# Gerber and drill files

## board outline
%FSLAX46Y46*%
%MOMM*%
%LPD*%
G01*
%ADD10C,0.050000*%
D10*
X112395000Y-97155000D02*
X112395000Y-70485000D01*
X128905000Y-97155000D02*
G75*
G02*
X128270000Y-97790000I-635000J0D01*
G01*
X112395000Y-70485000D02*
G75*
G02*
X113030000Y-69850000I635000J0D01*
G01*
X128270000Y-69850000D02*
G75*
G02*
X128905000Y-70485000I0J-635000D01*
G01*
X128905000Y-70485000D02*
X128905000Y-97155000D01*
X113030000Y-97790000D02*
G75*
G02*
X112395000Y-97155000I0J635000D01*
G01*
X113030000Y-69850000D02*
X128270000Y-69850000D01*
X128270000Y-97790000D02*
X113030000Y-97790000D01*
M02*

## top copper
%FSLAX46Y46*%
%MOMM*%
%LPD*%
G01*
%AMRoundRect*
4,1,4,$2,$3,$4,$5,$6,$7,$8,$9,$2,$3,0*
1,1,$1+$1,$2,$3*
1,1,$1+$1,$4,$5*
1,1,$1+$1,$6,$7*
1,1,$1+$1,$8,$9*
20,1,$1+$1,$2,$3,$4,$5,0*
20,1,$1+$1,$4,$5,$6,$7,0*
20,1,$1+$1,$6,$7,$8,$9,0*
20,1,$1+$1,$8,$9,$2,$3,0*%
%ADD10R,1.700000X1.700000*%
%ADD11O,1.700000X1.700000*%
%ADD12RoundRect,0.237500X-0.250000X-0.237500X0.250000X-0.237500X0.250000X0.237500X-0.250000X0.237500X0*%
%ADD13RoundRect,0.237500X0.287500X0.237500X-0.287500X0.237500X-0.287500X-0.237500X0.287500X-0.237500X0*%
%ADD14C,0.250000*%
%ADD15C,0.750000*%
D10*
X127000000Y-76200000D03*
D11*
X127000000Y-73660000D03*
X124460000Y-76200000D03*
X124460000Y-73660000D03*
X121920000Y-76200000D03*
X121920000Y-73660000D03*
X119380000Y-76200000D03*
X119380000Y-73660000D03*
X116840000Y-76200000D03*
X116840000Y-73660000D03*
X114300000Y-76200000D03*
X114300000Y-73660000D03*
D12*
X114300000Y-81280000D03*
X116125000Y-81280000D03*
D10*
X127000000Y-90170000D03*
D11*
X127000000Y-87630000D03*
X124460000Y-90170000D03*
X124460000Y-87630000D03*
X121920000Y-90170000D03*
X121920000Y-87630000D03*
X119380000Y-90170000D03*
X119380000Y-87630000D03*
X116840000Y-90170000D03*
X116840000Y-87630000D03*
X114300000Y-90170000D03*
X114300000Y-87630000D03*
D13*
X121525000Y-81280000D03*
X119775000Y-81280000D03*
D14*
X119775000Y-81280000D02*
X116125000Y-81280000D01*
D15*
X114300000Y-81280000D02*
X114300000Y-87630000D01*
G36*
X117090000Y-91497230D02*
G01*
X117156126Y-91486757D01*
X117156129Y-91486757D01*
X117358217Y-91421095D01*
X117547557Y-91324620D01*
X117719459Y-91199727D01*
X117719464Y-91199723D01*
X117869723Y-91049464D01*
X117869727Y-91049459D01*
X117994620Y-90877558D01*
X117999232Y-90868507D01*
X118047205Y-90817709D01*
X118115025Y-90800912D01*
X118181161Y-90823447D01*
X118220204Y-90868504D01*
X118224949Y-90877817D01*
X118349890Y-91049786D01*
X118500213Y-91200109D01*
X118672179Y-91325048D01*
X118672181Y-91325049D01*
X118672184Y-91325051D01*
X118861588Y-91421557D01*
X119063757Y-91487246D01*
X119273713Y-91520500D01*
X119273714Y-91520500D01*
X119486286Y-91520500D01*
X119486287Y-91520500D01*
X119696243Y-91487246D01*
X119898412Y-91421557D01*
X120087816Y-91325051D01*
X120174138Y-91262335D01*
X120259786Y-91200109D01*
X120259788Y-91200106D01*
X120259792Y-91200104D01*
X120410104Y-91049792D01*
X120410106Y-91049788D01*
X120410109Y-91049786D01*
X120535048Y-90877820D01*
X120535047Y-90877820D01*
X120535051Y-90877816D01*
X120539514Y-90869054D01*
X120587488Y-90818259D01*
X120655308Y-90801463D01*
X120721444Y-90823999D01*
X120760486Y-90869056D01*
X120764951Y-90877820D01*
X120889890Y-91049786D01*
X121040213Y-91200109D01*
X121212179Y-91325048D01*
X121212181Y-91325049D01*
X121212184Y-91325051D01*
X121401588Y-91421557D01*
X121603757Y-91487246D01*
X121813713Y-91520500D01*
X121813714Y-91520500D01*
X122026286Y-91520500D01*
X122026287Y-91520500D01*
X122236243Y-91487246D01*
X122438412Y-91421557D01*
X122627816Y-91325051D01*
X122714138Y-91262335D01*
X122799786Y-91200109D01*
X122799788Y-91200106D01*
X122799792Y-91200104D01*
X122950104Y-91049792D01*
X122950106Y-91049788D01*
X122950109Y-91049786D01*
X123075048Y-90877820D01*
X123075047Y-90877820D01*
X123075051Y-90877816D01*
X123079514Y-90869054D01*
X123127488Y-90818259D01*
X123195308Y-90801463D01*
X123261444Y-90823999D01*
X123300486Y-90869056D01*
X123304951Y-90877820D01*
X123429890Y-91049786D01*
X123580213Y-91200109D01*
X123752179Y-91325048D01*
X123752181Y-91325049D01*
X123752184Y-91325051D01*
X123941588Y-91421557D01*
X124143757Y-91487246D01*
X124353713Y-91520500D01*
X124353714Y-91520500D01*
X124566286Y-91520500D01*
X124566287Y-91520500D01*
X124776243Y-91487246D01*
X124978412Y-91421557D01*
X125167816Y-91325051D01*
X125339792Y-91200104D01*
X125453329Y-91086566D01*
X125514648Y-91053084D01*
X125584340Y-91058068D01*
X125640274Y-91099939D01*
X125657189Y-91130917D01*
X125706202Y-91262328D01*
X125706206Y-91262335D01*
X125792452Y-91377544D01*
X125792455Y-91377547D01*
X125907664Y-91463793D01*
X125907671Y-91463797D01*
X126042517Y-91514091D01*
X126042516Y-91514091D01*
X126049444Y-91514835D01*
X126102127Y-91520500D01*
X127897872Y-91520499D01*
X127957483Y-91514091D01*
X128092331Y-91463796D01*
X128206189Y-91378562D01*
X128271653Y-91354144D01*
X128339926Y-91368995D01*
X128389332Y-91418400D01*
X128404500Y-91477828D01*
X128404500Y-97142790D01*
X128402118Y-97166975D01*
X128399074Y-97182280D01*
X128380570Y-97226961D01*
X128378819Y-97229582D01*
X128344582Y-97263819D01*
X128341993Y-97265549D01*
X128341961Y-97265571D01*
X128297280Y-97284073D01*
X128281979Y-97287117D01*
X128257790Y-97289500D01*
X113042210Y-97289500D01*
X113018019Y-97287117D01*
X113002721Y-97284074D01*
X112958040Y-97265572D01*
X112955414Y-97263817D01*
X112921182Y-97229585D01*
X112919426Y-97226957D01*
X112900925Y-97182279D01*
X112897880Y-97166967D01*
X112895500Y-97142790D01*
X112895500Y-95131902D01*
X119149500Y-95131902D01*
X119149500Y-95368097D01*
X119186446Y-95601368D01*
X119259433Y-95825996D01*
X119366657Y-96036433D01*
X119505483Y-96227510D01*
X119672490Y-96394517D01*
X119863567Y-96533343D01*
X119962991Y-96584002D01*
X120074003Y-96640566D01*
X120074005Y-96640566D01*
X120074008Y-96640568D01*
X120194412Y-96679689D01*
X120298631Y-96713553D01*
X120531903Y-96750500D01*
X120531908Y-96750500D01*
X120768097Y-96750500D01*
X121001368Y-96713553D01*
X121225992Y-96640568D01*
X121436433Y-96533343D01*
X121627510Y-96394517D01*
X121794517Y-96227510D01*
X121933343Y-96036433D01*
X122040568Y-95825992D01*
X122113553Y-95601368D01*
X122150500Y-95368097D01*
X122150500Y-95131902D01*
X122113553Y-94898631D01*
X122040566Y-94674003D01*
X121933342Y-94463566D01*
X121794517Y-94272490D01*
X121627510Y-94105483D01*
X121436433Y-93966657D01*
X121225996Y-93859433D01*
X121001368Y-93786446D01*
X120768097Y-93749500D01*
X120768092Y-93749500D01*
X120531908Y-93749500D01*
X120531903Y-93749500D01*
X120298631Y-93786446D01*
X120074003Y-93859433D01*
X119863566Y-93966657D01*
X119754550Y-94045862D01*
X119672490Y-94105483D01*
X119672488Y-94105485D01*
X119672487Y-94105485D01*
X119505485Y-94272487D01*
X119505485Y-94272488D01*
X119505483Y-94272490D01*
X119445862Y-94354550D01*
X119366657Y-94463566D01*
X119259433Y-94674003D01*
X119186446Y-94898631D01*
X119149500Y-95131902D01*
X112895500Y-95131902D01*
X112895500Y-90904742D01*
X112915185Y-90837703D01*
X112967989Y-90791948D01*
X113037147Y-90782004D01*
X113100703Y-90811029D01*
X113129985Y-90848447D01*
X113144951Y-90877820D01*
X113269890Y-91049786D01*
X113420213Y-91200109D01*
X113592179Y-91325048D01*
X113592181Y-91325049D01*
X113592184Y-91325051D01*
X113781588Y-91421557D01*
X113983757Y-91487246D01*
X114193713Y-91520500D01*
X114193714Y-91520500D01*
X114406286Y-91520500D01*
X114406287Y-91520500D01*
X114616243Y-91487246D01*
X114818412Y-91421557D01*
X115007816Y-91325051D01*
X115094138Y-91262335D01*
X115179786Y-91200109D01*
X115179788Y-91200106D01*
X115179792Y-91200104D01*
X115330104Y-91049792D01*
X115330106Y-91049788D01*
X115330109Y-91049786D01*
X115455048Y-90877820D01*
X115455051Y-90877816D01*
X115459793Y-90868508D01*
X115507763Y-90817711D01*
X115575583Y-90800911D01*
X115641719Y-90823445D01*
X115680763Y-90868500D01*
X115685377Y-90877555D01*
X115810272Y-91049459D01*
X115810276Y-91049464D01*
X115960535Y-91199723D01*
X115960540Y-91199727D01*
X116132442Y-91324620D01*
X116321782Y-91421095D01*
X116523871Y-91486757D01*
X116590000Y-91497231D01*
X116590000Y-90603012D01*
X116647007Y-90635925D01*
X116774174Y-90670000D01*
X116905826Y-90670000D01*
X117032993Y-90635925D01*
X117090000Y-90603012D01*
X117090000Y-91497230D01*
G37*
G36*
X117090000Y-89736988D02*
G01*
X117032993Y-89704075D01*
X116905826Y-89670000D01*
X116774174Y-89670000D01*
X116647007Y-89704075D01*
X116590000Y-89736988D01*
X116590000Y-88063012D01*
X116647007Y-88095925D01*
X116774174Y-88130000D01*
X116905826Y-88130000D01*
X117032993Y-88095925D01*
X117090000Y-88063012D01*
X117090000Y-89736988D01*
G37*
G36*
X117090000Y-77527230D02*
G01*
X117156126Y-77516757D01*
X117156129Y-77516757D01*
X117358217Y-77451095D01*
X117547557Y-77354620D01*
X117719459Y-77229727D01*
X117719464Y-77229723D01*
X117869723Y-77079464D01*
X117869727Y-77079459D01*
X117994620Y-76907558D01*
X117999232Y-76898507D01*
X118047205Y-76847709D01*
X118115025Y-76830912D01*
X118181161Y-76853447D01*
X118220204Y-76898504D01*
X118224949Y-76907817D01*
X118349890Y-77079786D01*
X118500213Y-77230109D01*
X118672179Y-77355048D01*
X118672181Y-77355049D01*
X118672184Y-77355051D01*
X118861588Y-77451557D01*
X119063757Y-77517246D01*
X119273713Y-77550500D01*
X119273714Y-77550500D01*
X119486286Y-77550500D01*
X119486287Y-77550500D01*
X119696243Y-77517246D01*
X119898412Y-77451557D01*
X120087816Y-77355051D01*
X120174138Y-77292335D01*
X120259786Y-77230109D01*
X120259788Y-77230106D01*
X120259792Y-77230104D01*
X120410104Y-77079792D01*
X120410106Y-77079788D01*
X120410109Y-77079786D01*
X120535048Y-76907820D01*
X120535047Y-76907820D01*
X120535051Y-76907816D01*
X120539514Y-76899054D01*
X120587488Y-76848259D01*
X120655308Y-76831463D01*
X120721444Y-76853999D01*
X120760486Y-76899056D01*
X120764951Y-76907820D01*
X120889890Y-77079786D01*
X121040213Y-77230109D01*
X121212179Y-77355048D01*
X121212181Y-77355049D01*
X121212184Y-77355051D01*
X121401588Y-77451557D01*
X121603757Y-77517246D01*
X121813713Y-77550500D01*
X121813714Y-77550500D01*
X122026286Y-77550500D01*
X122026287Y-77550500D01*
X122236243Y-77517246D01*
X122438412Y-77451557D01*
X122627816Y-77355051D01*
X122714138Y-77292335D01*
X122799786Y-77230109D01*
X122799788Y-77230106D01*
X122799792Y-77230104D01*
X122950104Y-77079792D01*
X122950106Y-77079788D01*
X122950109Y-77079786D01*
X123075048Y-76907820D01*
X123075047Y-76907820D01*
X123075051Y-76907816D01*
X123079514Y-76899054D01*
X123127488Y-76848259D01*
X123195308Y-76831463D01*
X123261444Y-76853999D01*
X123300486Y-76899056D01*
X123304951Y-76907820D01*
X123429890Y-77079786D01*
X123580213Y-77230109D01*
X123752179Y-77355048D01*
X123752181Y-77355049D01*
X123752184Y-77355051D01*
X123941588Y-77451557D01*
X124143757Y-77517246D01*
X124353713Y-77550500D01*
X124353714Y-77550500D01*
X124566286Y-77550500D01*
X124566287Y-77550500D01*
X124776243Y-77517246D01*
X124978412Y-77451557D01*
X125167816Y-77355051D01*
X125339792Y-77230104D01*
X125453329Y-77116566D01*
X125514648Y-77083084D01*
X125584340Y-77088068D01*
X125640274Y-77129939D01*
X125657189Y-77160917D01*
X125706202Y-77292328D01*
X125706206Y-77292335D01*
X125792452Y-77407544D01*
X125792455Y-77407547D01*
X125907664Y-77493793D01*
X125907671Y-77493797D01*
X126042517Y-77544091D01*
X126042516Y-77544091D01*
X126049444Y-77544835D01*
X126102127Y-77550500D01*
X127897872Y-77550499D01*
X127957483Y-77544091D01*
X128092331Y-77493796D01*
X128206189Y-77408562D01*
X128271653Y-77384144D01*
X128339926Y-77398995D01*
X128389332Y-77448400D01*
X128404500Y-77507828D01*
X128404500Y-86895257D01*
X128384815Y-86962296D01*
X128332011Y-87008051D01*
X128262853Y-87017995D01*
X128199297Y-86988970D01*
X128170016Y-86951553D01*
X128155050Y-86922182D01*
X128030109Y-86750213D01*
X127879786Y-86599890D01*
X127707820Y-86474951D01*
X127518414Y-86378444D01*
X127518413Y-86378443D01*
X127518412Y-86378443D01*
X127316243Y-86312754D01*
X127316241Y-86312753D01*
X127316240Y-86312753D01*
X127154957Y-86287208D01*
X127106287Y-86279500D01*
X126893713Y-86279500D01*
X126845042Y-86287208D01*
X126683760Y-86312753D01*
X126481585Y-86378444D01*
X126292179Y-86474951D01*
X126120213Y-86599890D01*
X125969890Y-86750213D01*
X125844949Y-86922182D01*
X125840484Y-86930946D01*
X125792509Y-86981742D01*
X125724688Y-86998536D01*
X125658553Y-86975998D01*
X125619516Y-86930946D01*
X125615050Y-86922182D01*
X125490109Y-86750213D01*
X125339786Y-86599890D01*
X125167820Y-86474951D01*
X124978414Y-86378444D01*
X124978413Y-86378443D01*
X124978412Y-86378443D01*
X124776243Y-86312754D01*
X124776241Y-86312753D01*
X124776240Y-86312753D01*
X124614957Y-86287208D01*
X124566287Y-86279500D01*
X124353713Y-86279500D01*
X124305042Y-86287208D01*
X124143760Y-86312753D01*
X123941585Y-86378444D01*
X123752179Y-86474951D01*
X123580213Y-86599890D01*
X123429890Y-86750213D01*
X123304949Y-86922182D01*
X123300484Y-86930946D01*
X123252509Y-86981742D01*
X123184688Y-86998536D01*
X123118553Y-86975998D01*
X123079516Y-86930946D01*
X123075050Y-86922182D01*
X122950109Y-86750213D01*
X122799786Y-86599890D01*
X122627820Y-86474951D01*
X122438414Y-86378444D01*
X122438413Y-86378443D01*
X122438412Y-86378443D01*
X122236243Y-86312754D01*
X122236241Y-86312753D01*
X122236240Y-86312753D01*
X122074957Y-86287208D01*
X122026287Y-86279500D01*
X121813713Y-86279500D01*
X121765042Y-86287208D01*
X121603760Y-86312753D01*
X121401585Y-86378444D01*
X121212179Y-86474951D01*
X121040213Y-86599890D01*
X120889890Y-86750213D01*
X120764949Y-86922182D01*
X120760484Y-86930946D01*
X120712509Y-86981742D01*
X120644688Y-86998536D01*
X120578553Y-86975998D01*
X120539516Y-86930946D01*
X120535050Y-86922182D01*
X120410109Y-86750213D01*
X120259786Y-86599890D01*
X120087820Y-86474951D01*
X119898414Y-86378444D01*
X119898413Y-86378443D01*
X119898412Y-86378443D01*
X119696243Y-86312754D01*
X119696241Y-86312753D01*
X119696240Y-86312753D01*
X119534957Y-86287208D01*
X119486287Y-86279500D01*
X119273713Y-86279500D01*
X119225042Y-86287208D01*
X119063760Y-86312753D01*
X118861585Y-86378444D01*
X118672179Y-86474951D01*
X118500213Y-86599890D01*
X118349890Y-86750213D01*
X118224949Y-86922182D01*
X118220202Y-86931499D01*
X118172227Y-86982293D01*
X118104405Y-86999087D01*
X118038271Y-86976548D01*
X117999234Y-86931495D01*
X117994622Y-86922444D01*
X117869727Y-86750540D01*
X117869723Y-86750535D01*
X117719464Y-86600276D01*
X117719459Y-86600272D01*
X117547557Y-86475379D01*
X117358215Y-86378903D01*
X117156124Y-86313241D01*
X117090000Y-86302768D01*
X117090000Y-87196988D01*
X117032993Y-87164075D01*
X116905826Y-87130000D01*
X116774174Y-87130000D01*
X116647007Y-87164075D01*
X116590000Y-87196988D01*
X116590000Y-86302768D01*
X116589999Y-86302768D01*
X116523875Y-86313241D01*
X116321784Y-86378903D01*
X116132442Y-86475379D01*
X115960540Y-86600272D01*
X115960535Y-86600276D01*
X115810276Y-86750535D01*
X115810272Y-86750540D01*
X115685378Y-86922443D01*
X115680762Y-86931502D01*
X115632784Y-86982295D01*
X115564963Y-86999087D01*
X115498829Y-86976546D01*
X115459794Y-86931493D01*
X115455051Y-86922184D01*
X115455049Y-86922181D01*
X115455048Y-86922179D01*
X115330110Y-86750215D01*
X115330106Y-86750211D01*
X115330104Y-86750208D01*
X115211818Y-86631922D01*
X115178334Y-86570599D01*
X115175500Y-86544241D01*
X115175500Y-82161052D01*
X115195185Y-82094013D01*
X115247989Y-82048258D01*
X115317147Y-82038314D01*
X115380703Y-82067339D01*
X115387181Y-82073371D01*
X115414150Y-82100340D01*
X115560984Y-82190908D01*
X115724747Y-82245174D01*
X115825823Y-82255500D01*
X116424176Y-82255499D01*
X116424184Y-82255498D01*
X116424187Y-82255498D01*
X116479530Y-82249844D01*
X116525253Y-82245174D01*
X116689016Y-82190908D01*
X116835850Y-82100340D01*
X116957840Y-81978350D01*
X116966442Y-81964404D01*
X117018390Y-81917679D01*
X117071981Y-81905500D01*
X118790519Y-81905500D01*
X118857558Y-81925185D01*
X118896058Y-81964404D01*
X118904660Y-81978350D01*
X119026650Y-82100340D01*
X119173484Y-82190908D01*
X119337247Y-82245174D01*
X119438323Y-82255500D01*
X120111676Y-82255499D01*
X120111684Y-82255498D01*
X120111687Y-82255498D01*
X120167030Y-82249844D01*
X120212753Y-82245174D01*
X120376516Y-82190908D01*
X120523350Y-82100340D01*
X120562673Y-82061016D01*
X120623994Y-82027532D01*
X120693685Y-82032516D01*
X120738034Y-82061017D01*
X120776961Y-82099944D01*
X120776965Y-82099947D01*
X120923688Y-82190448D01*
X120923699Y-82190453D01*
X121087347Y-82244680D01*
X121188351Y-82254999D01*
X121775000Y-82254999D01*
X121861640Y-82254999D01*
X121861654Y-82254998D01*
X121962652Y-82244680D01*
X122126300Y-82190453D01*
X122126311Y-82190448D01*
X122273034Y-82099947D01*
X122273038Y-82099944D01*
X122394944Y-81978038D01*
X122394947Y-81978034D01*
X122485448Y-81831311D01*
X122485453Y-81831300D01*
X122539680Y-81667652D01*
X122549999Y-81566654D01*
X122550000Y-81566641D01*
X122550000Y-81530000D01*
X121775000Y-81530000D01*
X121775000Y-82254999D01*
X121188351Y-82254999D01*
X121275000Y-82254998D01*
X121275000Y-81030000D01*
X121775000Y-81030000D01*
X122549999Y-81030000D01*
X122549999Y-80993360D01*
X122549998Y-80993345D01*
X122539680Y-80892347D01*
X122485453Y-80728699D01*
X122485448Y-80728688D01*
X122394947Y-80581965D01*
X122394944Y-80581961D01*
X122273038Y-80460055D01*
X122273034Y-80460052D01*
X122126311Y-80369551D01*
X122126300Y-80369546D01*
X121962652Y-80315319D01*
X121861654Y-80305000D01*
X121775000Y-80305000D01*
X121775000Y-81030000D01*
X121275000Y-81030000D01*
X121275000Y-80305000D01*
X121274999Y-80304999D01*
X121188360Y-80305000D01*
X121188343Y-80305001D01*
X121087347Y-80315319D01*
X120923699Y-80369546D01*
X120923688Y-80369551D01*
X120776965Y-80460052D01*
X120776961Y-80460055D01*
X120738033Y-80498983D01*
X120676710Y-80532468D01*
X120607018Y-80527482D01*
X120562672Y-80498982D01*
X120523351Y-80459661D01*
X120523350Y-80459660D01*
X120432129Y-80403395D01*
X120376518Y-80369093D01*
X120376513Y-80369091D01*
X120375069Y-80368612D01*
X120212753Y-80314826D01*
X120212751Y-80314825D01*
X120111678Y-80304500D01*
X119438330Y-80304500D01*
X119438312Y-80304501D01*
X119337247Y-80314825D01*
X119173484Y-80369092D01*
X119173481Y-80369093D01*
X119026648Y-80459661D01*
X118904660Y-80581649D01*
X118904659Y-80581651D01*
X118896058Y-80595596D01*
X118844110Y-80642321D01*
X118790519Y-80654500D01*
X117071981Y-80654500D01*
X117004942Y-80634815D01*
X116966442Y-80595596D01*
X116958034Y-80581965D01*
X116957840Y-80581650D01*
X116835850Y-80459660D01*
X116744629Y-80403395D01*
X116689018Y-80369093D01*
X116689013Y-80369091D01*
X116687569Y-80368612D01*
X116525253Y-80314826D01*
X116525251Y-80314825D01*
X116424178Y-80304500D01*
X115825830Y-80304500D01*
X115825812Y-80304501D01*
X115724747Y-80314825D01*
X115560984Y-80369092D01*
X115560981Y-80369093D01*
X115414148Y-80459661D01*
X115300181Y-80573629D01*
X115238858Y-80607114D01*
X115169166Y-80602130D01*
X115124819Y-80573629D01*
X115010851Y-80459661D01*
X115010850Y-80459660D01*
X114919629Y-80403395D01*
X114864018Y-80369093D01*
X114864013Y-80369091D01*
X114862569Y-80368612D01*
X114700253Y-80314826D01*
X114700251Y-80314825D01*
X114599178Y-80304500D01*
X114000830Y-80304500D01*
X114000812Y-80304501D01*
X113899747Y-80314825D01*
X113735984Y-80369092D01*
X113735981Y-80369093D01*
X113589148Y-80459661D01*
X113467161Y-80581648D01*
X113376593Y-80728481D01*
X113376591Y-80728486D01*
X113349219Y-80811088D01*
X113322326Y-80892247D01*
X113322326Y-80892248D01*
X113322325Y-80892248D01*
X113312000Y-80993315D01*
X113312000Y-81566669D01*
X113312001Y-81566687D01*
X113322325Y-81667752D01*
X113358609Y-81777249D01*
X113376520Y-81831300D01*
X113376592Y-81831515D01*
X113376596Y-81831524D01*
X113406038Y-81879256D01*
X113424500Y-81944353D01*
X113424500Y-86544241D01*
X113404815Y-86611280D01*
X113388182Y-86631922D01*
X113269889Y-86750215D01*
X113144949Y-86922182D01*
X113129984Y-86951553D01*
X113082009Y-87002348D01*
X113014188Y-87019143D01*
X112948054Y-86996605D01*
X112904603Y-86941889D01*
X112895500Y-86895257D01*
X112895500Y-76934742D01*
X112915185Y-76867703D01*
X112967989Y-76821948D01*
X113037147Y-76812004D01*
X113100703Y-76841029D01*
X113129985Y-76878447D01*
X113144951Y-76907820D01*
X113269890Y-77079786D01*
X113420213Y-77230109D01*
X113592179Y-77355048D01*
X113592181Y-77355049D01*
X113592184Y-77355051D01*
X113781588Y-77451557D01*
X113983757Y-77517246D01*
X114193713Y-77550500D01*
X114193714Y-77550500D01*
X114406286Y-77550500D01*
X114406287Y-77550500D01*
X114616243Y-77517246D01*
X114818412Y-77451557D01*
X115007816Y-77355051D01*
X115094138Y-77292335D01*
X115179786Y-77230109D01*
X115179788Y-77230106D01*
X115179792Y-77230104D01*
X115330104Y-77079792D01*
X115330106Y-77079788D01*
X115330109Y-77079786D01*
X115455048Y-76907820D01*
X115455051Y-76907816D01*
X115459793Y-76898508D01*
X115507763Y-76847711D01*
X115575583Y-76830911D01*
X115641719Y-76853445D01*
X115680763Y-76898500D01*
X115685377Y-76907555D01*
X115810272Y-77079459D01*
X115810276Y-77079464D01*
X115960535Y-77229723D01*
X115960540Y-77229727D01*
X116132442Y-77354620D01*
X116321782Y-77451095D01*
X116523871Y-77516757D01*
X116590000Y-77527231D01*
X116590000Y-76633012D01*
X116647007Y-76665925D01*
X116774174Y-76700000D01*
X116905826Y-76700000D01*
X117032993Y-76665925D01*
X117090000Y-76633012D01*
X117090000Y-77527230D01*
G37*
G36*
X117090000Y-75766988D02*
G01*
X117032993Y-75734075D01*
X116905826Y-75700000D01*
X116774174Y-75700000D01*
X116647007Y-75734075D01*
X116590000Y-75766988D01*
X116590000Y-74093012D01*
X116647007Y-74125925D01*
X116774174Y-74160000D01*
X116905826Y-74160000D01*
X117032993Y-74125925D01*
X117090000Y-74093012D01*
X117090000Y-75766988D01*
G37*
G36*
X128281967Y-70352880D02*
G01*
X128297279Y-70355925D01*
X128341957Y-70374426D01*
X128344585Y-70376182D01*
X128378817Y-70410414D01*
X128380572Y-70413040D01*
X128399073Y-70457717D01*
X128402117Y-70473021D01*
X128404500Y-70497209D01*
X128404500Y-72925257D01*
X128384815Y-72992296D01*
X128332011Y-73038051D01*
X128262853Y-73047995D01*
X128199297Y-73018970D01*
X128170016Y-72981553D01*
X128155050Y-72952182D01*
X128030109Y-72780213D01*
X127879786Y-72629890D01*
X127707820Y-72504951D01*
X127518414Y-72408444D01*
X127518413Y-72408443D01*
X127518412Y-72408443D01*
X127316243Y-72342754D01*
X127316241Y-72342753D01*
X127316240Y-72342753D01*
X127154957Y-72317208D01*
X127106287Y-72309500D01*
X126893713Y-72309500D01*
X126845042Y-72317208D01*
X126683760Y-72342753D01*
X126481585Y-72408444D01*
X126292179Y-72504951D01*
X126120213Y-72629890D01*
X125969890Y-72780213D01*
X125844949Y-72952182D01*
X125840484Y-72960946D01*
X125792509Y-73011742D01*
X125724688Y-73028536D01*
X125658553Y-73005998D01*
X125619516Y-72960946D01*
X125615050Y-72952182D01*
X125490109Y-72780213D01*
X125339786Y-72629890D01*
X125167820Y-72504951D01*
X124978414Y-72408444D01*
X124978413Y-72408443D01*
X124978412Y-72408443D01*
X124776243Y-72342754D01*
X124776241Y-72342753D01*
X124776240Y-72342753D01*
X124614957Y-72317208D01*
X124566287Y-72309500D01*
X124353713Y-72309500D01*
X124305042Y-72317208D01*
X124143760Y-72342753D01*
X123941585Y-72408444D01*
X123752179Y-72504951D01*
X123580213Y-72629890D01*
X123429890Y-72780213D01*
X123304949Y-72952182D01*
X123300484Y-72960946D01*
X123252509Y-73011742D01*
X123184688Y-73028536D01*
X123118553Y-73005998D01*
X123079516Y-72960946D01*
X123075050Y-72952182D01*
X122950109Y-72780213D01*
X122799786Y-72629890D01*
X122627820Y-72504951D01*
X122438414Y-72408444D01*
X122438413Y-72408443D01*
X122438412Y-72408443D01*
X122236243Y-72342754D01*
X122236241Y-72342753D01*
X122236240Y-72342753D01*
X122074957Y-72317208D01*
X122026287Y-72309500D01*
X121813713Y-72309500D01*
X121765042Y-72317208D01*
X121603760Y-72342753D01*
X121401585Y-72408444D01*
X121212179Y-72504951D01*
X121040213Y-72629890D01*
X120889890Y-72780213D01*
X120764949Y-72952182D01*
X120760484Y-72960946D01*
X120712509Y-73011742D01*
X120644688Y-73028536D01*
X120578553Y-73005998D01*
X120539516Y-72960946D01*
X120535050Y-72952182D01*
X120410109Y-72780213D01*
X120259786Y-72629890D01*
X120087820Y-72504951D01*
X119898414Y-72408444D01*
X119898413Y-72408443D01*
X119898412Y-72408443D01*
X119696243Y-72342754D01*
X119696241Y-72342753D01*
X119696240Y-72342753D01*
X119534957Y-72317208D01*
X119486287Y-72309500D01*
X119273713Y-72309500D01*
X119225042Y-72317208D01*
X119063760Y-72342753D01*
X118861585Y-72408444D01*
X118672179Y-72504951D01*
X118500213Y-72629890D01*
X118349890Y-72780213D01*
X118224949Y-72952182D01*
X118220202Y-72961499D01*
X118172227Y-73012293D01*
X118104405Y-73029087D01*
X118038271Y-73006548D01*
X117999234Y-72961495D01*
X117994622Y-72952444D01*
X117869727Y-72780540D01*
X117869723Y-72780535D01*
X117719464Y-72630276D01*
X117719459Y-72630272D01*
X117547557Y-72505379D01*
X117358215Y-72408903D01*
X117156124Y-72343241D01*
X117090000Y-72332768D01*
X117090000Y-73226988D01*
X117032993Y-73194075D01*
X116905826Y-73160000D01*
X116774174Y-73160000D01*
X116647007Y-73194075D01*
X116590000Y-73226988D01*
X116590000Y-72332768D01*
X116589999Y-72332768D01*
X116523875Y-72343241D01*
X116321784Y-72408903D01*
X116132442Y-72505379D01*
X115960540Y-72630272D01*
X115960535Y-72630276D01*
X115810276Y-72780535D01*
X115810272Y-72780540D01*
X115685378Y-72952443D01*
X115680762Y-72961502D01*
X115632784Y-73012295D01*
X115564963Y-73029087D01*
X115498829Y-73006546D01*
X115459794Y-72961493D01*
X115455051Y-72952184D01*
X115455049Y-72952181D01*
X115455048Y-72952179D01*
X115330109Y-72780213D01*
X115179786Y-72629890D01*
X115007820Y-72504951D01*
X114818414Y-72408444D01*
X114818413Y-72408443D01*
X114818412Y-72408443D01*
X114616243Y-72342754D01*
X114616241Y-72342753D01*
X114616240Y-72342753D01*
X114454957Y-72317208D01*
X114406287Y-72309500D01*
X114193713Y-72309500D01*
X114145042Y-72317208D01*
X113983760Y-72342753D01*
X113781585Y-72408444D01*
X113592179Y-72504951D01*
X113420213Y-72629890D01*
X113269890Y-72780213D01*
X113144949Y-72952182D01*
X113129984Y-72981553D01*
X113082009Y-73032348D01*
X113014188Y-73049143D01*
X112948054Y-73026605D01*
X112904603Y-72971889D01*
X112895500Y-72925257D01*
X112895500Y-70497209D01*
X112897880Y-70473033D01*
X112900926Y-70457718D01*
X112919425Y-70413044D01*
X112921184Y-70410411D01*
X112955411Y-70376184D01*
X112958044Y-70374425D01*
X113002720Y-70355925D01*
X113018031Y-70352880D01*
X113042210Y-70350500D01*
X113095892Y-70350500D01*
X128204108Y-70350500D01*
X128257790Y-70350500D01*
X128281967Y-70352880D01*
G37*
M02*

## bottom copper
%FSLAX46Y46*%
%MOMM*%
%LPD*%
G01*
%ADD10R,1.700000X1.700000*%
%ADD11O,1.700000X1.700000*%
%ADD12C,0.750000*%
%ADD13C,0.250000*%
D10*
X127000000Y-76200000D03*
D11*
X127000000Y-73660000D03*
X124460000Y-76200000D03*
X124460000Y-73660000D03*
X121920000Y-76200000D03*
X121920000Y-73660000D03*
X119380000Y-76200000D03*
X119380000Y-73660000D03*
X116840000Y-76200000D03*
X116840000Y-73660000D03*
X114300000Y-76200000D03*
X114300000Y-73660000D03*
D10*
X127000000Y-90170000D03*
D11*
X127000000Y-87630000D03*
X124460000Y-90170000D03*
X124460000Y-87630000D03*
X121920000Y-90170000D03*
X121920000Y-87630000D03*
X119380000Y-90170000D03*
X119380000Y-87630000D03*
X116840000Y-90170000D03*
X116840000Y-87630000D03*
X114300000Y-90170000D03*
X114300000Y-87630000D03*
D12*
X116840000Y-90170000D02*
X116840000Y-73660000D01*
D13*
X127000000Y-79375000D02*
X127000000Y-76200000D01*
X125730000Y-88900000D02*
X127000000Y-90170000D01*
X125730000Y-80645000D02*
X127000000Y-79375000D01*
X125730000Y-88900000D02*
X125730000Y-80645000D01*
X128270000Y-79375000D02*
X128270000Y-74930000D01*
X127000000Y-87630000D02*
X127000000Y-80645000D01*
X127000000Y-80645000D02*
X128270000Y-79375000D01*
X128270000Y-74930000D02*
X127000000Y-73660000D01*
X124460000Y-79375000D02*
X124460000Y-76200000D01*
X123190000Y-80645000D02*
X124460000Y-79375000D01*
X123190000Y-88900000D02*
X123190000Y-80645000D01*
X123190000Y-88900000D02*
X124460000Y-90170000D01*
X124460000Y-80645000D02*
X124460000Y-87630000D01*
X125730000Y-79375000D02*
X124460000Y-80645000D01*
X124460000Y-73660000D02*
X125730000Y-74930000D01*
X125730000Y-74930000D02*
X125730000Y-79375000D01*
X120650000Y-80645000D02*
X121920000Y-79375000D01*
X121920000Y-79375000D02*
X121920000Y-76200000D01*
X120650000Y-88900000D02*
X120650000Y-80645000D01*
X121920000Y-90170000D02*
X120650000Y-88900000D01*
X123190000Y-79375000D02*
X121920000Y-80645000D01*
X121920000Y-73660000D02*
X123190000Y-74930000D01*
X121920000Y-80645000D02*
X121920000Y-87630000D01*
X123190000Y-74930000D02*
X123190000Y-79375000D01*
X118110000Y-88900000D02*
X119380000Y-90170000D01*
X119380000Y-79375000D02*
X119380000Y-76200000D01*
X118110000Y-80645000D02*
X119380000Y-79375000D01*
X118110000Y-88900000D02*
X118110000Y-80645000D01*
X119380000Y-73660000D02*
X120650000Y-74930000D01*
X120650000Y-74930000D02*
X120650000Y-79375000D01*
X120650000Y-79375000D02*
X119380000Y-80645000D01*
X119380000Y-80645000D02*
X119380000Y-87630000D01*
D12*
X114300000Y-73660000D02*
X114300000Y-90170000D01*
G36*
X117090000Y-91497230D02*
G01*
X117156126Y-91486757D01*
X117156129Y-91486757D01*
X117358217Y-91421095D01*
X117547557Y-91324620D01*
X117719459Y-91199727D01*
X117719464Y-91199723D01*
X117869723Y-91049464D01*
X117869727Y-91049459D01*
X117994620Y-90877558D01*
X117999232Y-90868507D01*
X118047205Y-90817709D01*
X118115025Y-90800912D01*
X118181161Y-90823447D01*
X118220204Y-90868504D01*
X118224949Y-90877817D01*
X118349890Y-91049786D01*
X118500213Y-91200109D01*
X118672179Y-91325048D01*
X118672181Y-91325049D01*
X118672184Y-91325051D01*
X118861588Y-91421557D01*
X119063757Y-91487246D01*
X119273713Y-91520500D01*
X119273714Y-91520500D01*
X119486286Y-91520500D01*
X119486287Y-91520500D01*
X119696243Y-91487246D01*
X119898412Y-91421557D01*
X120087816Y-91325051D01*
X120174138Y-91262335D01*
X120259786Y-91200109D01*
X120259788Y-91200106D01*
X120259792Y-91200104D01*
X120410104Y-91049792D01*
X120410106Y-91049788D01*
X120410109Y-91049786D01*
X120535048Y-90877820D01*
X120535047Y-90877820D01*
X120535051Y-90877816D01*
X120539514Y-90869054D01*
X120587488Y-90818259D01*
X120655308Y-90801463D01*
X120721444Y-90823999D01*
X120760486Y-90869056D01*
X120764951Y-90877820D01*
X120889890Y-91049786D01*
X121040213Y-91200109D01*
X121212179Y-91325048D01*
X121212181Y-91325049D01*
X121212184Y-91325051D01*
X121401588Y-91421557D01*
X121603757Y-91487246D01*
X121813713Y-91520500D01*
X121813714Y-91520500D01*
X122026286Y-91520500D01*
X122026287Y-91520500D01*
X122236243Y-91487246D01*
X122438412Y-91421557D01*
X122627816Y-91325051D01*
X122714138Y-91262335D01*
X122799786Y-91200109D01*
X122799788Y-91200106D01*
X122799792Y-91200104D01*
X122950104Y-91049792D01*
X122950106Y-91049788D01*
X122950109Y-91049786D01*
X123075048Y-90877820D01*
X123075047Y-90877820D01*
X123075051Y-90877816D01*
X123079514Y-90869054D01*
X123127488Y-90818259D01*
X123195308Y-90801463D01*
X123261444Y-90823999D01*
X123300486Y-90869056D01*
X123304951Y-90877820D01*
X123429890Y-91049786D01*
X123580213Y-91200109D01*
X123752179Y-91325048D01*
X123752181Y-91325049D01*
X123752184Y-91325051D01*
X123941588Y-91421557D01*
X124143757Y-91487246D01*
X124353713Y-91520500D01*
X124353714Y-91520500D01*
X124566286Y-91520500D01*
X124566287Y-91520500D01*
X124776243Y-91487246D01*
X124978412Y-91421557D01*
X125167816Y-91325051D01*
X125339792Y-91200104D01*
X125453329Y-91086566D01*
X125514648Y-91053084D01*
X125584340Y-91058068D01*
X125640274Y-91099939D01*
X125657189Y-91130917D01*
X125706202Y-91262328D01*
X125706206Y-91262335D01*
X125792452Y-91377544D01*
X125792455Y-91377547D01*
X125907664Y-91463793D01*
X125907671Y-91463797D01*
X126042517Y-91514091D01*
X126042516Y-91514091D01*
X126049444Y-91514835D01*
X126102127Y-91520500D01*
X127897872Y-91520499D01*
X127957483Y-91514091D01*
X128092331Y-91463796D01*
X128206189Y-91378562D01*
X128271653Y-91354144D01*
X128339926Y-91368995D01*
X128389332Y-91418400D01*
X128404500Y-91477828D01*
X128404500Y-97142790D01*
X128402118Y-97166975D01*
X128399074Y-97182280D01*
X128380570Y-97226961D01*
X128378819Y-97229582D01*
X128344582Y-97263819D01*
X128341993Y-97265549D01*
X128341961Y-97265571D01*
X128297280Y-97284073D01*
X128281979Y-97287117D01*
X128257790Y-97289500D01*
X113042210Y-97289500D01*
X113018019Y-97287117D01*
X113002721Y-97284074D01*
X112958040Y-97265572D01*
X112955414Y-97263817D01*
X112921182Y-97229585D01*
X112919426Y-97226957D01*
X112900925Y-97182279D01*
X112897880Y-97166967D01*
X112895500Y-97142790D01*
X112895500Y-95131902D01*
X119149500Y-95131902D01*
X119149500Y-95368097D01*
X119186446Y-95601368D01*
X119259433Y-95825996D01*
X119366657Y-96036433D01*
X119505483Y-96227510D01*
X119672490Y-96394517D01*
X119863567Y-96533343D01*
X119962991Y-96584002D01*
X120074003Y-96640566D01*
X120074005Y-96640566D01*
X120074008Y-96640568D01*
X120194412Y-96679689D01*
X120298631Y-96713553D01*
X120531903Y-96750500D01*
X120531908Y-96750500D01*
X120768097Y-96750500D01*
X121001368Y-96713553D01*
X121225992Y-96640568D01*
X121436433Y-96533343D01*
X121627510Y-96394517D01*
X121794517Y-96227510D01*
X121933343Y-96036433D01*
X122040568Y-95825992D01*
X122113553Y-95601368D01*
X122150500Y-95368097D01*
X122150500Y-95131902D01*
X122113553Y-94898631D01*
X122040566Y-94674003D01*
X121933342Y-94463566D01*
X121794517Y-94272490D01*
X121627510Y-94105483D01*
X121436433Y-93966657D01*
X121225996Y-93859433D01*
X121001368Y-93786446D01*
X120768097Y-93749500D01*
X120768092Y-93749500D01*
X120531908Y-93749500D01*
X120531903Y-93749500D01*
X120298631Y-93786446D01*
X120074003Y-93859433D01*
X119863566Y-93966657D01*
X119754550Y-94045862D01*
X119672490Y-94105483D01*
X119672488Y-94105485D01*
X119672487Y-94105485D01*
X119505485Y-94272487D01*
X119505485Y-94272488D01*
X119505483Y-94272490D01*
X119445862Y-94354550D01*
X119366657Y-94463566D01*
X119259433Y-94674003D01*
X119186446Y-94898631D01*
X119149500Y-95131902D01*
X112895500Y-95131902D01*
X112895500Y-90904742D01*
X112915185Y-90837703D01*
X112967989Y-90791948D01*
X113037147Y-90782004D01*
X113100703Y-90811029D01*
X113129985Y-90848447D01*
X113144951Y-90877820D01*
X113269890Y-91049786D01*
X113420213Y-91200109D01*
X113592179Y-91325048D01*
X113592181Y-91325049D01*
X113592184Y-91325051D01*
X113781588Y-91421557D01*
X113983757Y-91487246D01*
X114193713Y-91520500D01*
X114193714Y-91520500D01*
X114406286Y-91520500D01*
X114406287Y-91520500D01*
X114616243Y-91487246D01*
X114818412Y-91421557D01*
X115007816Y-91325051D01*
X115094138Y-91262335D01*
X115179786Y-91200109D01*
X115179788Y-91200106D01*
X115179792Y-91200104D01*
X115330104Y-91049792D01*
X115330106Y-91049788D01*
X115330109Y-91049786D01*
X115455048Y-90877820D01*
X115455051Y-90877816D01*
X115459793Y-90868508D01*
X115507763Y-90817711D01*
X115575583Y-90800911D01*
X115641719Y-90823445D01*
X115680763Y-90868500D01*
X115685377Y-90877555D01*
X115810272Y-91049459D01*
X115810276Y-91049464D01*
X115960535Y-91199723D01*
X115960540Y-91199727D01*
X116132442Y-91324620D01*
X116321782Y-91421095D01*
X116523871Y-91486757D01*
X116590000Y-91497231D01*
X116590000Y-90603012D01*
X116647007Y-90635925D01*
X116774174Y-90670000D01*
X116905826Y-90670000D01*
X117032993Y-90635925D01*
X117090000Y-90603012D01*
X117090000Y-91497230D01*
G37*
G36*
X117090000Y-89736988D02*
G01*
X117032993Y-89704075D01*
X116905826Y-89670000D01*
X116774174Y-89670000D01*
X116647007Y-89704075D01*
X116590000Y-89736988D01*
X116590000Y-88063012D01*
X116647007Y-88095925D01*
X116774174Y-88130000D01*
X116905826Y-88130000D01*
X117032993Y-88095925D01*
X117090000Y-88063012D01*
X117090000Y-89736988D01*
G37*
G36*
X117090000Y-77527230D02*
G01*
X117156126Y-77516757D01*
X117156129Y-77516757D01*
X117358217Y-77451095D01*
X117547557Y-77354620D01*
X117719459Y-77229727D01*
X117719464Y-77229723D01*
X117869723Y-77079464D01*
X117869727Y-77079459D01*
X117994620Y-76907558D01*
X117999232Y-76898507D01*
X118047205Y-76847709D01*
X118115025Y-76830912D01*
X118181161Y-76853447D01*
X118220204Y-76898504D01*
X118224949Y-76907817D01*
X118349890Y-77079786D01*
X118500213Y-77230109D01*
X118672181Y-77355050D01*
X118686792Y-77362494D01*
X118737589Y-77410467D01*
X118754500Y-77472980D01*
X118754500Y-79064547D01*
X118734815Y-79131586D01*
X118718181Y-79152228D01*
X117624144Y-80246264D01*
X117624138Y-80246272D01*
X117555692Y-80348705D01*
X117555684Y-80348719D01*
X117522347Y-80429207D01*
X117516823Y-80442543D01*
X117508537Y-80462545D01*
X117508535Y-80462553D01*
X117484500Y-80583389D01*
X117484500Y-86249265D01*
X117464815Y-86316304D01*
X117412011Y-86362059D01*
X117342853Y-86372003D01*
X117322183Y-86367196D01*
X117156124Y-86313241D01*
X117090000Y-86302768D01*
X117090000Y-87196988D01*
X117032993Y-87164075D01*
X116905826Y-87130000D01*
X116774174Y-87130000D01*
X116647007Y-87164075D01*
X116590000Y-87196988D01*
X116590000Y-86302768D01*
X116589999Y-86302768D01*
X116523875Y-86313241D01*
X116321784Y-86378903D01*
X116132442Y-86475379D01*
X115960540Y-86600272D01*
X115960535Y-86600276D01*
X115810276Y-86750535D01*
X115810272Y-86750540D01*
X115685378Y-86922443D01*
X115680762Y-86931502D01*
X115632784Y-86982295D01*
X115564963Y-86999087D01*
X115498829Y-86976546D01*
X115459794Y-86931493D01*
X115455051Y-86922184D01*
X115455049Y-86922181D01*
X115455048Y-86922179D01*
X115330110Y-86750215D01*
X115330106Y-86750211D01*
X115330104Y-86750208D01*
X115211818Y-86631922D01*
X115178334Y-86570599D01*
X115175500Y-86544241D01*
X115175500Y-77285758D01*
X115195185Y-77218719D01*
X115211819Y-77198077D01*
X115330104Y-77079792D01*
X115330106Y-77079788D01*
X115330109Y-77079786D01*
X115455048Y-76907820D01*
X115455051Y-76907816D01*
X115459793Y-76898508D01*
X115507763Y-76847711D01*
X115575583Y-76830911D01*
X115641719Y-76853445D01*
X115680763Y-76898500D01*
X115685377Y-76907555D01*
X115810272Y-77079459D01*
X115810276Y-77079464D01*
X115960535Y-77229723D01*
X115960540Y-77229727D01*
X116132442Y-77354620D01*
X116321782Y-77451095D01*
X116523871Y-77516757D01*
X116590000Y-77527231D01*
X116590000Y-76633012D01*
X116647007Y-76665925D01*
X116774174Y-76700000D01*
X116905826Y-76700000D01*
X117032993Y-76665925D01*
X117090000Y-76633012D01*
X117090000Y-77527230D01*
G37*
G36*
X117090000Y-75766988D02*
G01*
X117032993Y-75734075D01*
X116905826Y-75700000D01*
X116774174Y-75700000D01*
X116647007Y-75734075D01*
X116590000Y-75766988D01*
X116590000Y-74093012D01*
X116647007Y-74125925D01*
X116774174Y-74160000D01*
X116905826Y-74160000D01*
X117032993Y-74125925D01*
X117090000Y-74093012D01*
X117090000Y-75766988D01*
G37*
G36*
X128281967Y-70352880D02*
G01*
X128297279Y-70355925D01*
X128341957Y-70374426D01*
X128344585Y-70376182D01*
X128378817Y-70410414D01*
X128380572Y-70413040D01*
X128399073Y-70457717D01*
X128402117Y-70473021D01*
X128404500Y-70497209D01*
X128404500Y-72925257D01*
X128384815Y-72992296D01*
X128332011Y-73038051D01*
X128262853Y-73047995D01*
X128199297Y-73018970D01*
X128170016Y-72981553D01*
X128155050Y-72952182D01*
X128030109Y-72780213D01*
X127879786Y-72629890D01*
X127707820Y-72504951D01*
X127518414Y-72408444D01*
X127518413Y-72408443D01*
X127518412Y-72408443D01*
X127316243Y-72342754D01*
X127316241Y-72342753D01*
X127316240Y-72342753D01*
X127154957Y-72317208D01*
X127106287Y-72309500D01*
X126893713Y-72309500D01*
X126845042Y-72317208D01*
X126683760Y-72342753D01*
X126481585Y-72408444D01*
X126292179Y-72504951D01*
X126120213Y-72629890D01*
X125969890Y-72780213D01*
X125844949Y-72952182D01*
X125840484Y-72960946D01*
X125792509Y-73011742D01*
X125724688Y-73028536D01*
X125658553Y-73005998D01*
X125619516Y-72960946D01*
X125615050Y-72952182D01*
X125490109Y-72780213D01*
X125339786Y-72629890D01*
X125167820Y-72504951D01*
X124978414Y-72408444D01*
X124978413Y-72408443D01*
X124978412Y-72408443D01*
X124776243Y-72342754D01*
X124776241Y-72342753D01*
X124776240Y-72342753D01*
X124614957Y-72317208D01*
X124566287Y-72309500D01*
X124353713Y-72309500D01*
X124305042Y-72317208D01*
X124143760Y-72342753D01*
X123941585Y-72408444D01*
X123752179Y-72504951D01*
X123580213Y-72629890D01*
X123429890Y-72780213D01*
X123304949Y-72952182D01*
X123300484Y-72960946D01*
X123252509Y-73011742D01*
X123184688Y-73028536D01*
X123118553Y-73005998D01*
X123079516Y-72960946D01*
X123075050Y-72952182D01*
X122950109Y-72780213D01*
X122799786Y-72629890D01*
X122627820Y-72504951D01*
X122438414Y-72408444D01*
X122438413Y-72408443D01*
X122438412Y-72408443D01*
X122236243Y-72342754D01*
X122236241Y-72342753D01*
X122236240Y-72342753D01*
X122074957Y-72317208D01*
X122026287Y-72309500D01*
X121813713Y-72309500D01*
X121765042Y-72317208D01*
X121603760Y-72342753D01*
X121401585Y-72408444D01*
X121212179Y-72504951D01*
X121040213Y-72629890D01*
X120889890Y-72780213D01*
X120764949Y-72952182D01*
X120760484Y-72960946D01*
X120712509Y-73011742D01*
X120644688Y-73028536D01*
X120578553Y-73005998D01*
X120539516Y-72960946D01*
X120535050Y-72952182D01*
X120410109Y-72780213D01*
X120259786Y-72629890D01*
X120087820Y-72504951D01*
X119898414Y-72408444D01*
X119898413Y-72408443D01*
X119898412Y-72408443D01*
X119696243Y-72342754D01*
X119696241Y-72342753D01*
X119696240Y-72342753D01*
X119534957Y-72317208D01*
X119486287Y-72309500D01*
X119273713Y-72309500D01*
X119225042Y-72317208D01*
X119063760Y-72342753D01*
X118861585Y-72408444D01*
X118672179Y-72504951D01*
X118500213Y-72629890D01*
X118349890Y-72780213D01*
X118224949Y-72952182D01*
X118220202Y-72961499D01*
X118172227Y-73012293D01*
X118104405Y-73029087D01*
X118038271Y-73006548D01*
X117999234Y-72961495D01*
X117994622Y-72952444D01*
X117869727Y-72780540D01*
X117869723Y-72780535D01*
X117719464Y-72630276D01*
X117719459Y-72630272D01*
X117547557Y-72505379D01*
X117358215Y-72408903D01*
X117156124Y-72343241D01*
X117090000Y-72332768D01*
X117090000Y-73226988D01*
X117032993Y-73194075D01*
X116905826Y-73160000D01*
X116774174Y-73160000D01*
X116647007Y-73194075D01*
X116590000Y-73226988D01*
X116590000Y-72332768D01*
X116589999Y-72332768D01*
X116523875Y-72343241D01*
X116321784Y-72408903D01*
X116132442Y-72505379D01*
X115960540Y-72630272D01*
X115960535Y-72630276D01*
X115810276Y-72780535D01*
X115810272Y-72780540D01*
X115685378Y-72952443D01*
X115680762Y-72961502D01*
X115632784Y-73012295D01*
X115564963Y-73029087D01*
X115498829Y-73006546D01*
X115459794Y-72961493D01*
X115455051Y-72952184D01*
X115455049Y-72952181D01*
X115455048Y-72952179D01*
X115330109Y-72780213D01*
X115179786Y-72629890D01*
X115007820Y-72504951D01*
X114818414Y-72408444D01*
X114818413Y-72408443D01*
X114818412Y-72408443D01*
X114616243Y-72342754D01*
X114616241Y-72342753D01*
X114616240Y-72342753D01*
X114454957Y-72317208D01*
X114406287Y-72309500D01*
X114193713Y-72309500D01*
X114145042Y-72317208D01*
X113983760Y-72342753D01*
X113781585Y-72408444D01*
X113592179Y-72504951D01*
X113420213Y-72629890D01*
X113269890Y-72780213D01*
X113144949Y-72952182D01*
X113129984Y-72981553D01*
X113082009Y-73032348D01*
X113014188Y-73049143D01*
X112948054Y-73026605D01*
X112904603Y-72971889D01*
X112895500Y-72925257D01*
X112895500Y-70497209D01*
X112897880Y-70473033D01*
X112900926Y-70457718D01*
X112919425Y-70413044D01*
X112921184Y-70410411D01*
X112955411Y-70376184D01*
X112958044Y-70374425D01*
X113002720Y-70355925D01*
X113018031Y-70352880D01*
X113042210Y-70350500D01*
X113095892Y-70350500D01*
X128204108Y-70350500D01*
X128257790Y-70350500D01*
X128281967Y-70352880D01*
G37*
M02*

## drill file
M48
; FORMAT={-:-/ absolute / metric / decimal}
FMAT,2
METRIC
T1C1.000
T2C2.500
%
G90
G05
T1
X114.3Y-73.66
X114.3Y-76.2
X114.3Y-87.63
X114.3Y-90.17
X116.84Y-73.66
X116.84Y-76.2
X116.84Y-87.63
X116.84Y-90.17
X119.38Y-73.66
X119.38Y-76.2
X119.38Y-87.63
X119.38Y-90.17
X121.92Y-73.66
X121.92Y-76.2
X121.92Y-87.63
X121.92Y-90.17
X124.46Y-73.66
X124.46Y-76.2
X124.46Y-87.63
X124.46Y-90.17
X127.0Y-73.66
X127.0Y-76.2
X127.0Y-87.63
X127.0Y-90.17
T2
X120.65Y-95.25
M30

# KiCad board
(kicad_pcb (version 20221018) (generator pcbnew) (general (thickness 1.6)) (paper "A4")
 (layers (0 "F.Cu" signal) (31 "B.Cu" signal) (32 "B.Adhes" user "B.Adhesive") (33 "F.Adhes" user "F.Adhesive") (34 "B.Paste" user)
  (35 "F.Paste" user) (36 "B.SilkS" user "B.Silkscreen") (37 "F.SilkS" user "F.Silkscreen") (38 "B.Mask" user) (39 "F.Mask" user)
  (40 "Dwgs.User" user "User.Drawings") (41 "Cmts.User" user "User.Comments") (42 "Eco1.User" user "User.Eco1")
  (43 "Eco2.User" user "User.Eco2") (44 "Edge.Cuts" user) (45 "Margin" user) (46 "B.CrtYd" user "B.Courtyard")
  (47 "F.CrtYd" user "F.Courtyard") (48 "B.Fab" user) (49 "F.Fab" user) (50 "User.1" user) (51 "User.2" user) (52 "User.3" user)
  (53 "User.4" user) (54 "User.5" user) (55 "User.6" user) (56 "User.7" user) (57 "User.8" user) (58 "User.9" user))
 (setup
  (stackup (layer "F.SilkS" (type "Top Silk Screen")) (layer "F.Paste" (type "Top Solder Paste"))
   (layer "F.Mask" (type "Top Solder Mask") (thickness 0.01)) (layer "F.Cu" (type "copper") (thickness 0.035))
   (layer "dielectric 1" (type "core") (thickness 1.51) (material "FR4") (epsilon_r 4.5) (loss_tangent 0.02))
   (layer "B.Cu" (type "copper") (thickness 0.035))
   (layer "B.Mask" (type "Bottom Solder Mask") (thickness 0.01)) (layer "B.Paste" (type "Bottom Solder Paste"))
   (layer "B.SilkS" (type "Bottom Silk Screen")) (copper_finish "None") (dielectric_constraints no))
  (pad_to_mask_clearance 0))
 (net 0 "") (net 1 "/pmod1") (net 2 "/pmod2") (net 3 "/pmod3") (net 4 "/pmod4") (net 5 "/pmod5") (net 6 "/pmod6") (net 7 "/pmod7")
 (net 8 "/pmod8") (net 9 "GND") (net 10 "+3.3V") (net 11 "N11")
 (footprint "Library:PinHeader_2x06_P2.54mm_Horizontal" (layer "F.Cu") (at 127 76.2 90)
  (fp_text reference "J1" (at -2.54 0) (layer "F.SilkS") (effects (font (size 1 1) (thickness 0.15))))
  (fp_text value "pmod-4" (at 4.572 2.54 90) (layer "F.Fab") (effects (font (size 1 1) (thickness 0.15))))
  (pad "1" thru_hole rect (at 0 0 90) (size 1.7 1.7) (drill 1) (layers "*.Cu" "*.Mask") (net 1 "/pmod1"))
  (pad "2" thru_hole oval (at 2.54 0 90) (size 1.7 1.7) (drill 1) (layers "*.Cu" "*.Mask") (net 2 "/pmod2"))
  (pad "3" thru_hole oval (at 0 -2.54 90) (size 1.7 1.7) (drill 1) (layers "*.Cu" "*.Mask") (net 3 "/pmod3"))
  (pad "4" thru_hole oval (at 2.54 -2.54 90) (size 1.7 1.7) (drill 1) (layers "*.Cu" "*.Mask") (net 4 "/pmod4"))
  (pad "5" thru_hole oval (at 0 -5.08 90) (size 1.7 1.7) (drill 1) (layers "*.Cu" "*.Mask") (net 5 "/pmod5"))
  (pad "6" thru_hole oval (at 2.54 -5.08 90) (size 1.7 1.7) (drill 1) (layers "*.Cu" "*.Mask") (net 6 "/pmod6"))
  (pad "7" thru_hole oval (at 0 -7.62 90) (size 1.7 1.7) (drill 1) (layers "*.Cu" "*.Mask") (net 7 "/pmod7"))
  (pad "8" thru_hole oval (at 2.54 -7.62 90) (size 1.7 1.7) (drill 1) (layers "*.Cu" "*.Mask") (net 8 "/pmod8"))
  (pad "9" thru_hole oval (at 0 -10.16 90) (size 1.7 1.7) (drill 1) (layers "*.Cu" "*.Mask") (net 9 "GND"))
  (pad "10" thru_hole oval (at 2.54 -10.16 90) (size 1.7 1.7) (drill 1) (layers "*.Cu" "*.Mask") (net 9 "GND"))
  (pad "11" thru_hole oval (at 0 -12.7 90) (size 1.7 1.7) (drill 1) (layers "*.Cu" "*.Mask") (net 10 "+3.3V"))
  (pad "12" thru_hole oval (at 2.54 -12.7 90) (size 1.7 1.7) (drill 1) (layers "*.Cu" "*.Mask") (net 10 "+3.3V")))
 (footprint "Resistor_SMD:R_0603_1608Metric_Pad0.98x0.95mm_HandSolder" (layer "F.Cu") (at 115.2125 81.28)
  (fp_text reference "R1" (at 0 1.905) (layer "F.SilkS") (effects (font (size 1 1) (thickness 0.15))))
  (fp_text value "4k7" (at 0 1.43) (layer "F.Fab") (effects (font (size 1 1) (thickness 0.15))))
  (pad "1" smd roundrect (at -0.9125 0) (size 0.975 0.95) (layers "F.Cu" "F.Paste" "F.Mask") (roundrect_rratio 0.25) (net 10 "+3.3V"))
  (pad "2" smd roundrect (at 0.9125 0) (size 0.975 0.95) (layers "F.Cu" "F.Paste" "F.Mask") (roundrect_rratio 0.25) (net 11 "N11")))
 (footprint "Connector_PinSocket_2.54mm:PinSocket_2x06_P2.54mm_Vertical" (layer "F.Cu") (at 127 90.17 -90)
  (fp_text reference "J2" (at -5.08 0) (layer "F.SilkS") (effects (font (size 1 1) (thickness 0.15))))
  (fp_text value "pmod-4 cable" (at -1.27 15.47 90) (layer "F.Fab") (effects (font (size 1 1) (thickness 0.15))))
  (pad "1" thru_hole rect (at 0 0 270) (size 1.7 1.7) (drill 1) (layers "*.Cu" "*.Mask") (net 1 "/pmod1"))
  (pad "2" thru_hole oval (at -2.54 0 270) (size 1.7 1.7) (drill 1) (layers "*.Cu" "*.Mask") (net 2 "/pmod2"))
  (pad "3" thru_hole oval (at 0 2.54 270) (size 1.7 1.7) (drill 1) (layers "*.Cu" "*.Mask") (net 3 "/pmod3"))
  (pad "4" thru_hole oval (at -2.54 2.54 270) (size 1.7 1.7) (drill 1) (layers "*.Cu" "*.Mask") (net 4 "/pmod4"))
  (pad "5" thru_hole oval (at 0 5.08 270) (size 1.7 1.7) (drill 1) (layers "*.Cu" "*.Mask") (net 5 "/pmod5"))
  (pad "6" thru_hole oval (at -2.54 5.08 270) (size 1.7 1.7) (drill 1) (layers "*.Cu" "*.Mask") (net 6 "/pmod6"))
  (pad "7" thru_hole oval (at 0 7.62 270) (size 1.7 1.7) (drill 1) (layers "*.Cu" "*.Mask") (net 7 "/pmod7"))
  (pad "8" thru_hole oval (at -2.54 7.62 270) (size 1.7 1.7) (drill 1) (layers "*.Cu" "*.Mask") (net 8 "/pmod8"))
  (pad "9" thru_hole oval (at 0 10.16 270) (size 1.7 1.7) (drill 1) (layers "*.Cu" "*.Mask") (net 9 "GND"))
  (pad "10" thru_hole oval (at -2.54 10.16 270) (size 1.7 1.7) (drill 1) (layers "*.Cu" "*.Mask") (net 9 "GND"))
  (pad "11" thru_hole oval (at 0 12.7 270) (size 1.7 1.7) (drill 1) (layers "*.Cu" "*.Mask") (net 10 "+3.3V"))
  (pad "12" thru_hole oval (at -2.54 12.7 270) (size 1.7 1.7) (drill 1) (layers "*.Cu" "*.Mask") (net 10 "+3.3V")))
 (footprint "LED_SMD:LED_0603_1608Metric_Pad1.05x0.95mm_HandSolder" (layer "F.Cu") (at 120.65 81.28 180)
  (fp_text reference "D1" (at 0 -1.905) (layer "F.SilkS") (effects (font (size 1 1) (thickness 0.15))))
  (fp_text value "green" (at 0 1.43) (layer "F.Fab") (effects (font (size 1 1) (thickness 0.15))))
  (pad "1" smd roundrect (at -0.875 0 180) (size 1.05 0.95) (layers "F.Cu" "F.Paste" "F.Mask") (roundrect_rratio 0.25) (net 9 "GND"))
  (pad "2" smd roundrect (at 0.875 0 180) (size 1.05 0.95) (layers "F.Cu" "F.Paste" "F.Mask") (roundrect_rratio 0.25) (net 11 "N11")))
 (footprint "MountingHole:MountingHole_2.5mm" (layer "F.Cu") (at 120.65 95.25)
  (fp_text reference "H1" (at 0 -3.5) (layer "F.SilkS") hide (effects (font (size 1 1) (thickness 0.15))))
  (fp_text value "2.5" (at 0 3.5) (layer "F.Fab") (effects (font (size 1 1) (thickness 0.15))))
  (pad "" np_thru_hole circle (at 0 0) (size 2.5 2.5) (drill 2.5) (layers "*.Cu" "*.Mask")))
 (gr_line (start 112.395 97.155) (end 112.395 70.485) (stroke (width 0.05) (type default)) (layer "Edge.Cuts"))
 (gr_arc (start 128.905 97.155) (mid 128.719013 97.604013) (end 128.27 97.79) (stroke (width 0.05) (type default)) (layer "Edge.Cuts"))
 (gr_arc (start 112.395 70.485) (mid 112.580987 70.035987) (end 113.03 69.85) (stroke (width 0.05) (type default)) (layer "Edge.Cuts"))
 (gr_arc (start 128.27 69.85) (mid 128.719013 70.035987) (end 128.905 70.485) (stroke (width 0.05) (type default)) (layer "Edge.Cuts"))
 (gr_line (start 128.905 70.485) (end 128.905 97.155) (stroke (width 0.05) (type default)) (layer "Edge.Cuts"))
 (gr_arc (start 113.03 97.79) (mid 112.580987 97.604013) (end 112.395 97.155) (stroke (width 0.05) (type default)) (layer "Edge.Cuts"))
 (gr_line (start 113.03 69.85) (end 128.27 69.85) (stroke (width 0.05) (type default)) (layer "Edge.Cuts"))
 (gr_line (start 128.27 97.79) (end 113.03 97.79) (stroke (width 0.05) (type default)) (layer "Edge.Cuts"))
 (segment (start 116.84 90.17) (end 116.84 73.66) (width 0.75) (layer "B.Cu") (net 9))
 (segment (start 119.775 81.28) (end 116.125 81.28) (width 0.25) (layer "F.Cu") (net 11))
 (segment (start 127 79.375) (end 127 76.2) (width 0.25) (layer "B.Cu") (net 1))
 (segment (start 125.73 88.9) (end 127 90.17) (width 0.25) (layer "B.Cu") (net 1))
 (segment (start 125.73 80.645) (end 127 79.375) (width 0.25) (layer "B.Cu") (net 1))
 (segment (start 125.73 88.9) (end 125.73 80.645) (width 0.25) (layer "B.Cu") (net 1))
 (segment (start 128.27 79.375) (end 128.27 74.93) (width 0.25) (layer "B.Cu") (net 2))
 (segment (start 127 87.63) (end 127 80.645) (width 0.25) (layer "B.Cu") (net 2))
 (segment (start 127 80.645) (end 128.27 79.375) (width 0.25) (layer "B.Cu") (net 2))
 (segment (start 128.27 74.93) (end 127 73.66) (width 0.25) (layer "B.Cu") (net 2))
 (segment (start 124.46 79.375) (end 124.46 76.2) (width 0.25) (layer "B.Cu") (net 3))
 (segment (start 123.19 80.645) (end 124.46 79.375) (width 0.25) (layer "B.Cu") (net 3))
 (segment (start 123.19 88.9) (end 123.19 80.645) (width 0.25) (layer "B.Cu") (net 3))
 (segment (start 123.19 88.9) (end 124.46 90.17) (width 0.25) (layer "B.Cu") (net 3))
 (segment (start 124.46 80.645) (end 124.46 87.63) (width 0.25) (layer "B.Cu") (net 4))
 (segment (start 125.73 79.375) (end 124.46 80.645) (width 0.25) (layer "B.Cu") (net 4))
 (segment (start 124.46 73.66) (end 125.73 74.93) (width 0.25) (layer "B.Cu") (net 4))
 (segment (start 125.73 74.93) (end 125.73 79.375) (width 0.25) (layer "B.Cu") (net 4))
 (segment (start 120.65 80.645) (end 121.92 79.375) (width 0.25) (layer "B.Cu") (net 5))
 (segment (start 121.92 79.375) (end 121.92 76.2) (width 0.25) (layer "B.Cu") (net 5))
 (segment (start 120.65 88.9) (end 120.65 80.645) (width 0.25) (layer "B.Cu") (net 5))
 (segment (start 121.92 90.17) (end 120.65 88.9) (width 0.25) (layer "B.Cu") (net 5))
 (segment (start 123.19 79.375) (end 121.92 80.645) (width 0.25) (layer "B.Cu") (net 6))
 (segment (start 121.92 73.66) (end 123.19 74.93) (width 0.25) (layer "B.Cu") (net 6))
 (segment (start 121.92 80.645) (end 121.92 87.63) (width 0.25) (layer "B.Cu") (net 6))
 (segment (start 123.19 74.93) (end 123.19 79.375) (width 0.25) (layer "B.Cu") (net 6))
 (segment (start 118.11 88.9) (end 119.38 90.17) (width 0.25) (layer "B.Cu") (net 7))
 (segment (start 119.38 79.375) (end 119.38 76.2) (width 0.25) (layer "B.Cu") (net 7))
 (segment (start 118.11 80.645) (end 119.38 79.375) (width 0.25) (layer "B.Cu") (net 7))
 (segment (start 118.11 88.9) (end 118.11 80.645) (width 0.25) (layer "B.Cu") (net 7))
 (segment (start 119.38 73.66) (end 120.65 74.93) (width 0.25) (layer "B.Cu") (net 8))
 (segment (start 120.65 74.93) (end 120.65 79.375) (width 0.25) (layer "B.Cu") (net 8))
 (segment (start 120.65 79.375) (end 119.38 80.645) (width 0.25) (layer "B.Cu") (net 8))
 (segment (start 119.38 80.645) (end 119.38 87.63) (width 0.25) (layer "B.Cu") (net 8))
 (segment (start 114.3 81.28) (end 114.3 87.63) (width 0.75) (layer "F.Cu") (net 10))
 (segment (start 114.3 73.66) (end 114.3 90.17) (width 0.75) (layer "B.Cu") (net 10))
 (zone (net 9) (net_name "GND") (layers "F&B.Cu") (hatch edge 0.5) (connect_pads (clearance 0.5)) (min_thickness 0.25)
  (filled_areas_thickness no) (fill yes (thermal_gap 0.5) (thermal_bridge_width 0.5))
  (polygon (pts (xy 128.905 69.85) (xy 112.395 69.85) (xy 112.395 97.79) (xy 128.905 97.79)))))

